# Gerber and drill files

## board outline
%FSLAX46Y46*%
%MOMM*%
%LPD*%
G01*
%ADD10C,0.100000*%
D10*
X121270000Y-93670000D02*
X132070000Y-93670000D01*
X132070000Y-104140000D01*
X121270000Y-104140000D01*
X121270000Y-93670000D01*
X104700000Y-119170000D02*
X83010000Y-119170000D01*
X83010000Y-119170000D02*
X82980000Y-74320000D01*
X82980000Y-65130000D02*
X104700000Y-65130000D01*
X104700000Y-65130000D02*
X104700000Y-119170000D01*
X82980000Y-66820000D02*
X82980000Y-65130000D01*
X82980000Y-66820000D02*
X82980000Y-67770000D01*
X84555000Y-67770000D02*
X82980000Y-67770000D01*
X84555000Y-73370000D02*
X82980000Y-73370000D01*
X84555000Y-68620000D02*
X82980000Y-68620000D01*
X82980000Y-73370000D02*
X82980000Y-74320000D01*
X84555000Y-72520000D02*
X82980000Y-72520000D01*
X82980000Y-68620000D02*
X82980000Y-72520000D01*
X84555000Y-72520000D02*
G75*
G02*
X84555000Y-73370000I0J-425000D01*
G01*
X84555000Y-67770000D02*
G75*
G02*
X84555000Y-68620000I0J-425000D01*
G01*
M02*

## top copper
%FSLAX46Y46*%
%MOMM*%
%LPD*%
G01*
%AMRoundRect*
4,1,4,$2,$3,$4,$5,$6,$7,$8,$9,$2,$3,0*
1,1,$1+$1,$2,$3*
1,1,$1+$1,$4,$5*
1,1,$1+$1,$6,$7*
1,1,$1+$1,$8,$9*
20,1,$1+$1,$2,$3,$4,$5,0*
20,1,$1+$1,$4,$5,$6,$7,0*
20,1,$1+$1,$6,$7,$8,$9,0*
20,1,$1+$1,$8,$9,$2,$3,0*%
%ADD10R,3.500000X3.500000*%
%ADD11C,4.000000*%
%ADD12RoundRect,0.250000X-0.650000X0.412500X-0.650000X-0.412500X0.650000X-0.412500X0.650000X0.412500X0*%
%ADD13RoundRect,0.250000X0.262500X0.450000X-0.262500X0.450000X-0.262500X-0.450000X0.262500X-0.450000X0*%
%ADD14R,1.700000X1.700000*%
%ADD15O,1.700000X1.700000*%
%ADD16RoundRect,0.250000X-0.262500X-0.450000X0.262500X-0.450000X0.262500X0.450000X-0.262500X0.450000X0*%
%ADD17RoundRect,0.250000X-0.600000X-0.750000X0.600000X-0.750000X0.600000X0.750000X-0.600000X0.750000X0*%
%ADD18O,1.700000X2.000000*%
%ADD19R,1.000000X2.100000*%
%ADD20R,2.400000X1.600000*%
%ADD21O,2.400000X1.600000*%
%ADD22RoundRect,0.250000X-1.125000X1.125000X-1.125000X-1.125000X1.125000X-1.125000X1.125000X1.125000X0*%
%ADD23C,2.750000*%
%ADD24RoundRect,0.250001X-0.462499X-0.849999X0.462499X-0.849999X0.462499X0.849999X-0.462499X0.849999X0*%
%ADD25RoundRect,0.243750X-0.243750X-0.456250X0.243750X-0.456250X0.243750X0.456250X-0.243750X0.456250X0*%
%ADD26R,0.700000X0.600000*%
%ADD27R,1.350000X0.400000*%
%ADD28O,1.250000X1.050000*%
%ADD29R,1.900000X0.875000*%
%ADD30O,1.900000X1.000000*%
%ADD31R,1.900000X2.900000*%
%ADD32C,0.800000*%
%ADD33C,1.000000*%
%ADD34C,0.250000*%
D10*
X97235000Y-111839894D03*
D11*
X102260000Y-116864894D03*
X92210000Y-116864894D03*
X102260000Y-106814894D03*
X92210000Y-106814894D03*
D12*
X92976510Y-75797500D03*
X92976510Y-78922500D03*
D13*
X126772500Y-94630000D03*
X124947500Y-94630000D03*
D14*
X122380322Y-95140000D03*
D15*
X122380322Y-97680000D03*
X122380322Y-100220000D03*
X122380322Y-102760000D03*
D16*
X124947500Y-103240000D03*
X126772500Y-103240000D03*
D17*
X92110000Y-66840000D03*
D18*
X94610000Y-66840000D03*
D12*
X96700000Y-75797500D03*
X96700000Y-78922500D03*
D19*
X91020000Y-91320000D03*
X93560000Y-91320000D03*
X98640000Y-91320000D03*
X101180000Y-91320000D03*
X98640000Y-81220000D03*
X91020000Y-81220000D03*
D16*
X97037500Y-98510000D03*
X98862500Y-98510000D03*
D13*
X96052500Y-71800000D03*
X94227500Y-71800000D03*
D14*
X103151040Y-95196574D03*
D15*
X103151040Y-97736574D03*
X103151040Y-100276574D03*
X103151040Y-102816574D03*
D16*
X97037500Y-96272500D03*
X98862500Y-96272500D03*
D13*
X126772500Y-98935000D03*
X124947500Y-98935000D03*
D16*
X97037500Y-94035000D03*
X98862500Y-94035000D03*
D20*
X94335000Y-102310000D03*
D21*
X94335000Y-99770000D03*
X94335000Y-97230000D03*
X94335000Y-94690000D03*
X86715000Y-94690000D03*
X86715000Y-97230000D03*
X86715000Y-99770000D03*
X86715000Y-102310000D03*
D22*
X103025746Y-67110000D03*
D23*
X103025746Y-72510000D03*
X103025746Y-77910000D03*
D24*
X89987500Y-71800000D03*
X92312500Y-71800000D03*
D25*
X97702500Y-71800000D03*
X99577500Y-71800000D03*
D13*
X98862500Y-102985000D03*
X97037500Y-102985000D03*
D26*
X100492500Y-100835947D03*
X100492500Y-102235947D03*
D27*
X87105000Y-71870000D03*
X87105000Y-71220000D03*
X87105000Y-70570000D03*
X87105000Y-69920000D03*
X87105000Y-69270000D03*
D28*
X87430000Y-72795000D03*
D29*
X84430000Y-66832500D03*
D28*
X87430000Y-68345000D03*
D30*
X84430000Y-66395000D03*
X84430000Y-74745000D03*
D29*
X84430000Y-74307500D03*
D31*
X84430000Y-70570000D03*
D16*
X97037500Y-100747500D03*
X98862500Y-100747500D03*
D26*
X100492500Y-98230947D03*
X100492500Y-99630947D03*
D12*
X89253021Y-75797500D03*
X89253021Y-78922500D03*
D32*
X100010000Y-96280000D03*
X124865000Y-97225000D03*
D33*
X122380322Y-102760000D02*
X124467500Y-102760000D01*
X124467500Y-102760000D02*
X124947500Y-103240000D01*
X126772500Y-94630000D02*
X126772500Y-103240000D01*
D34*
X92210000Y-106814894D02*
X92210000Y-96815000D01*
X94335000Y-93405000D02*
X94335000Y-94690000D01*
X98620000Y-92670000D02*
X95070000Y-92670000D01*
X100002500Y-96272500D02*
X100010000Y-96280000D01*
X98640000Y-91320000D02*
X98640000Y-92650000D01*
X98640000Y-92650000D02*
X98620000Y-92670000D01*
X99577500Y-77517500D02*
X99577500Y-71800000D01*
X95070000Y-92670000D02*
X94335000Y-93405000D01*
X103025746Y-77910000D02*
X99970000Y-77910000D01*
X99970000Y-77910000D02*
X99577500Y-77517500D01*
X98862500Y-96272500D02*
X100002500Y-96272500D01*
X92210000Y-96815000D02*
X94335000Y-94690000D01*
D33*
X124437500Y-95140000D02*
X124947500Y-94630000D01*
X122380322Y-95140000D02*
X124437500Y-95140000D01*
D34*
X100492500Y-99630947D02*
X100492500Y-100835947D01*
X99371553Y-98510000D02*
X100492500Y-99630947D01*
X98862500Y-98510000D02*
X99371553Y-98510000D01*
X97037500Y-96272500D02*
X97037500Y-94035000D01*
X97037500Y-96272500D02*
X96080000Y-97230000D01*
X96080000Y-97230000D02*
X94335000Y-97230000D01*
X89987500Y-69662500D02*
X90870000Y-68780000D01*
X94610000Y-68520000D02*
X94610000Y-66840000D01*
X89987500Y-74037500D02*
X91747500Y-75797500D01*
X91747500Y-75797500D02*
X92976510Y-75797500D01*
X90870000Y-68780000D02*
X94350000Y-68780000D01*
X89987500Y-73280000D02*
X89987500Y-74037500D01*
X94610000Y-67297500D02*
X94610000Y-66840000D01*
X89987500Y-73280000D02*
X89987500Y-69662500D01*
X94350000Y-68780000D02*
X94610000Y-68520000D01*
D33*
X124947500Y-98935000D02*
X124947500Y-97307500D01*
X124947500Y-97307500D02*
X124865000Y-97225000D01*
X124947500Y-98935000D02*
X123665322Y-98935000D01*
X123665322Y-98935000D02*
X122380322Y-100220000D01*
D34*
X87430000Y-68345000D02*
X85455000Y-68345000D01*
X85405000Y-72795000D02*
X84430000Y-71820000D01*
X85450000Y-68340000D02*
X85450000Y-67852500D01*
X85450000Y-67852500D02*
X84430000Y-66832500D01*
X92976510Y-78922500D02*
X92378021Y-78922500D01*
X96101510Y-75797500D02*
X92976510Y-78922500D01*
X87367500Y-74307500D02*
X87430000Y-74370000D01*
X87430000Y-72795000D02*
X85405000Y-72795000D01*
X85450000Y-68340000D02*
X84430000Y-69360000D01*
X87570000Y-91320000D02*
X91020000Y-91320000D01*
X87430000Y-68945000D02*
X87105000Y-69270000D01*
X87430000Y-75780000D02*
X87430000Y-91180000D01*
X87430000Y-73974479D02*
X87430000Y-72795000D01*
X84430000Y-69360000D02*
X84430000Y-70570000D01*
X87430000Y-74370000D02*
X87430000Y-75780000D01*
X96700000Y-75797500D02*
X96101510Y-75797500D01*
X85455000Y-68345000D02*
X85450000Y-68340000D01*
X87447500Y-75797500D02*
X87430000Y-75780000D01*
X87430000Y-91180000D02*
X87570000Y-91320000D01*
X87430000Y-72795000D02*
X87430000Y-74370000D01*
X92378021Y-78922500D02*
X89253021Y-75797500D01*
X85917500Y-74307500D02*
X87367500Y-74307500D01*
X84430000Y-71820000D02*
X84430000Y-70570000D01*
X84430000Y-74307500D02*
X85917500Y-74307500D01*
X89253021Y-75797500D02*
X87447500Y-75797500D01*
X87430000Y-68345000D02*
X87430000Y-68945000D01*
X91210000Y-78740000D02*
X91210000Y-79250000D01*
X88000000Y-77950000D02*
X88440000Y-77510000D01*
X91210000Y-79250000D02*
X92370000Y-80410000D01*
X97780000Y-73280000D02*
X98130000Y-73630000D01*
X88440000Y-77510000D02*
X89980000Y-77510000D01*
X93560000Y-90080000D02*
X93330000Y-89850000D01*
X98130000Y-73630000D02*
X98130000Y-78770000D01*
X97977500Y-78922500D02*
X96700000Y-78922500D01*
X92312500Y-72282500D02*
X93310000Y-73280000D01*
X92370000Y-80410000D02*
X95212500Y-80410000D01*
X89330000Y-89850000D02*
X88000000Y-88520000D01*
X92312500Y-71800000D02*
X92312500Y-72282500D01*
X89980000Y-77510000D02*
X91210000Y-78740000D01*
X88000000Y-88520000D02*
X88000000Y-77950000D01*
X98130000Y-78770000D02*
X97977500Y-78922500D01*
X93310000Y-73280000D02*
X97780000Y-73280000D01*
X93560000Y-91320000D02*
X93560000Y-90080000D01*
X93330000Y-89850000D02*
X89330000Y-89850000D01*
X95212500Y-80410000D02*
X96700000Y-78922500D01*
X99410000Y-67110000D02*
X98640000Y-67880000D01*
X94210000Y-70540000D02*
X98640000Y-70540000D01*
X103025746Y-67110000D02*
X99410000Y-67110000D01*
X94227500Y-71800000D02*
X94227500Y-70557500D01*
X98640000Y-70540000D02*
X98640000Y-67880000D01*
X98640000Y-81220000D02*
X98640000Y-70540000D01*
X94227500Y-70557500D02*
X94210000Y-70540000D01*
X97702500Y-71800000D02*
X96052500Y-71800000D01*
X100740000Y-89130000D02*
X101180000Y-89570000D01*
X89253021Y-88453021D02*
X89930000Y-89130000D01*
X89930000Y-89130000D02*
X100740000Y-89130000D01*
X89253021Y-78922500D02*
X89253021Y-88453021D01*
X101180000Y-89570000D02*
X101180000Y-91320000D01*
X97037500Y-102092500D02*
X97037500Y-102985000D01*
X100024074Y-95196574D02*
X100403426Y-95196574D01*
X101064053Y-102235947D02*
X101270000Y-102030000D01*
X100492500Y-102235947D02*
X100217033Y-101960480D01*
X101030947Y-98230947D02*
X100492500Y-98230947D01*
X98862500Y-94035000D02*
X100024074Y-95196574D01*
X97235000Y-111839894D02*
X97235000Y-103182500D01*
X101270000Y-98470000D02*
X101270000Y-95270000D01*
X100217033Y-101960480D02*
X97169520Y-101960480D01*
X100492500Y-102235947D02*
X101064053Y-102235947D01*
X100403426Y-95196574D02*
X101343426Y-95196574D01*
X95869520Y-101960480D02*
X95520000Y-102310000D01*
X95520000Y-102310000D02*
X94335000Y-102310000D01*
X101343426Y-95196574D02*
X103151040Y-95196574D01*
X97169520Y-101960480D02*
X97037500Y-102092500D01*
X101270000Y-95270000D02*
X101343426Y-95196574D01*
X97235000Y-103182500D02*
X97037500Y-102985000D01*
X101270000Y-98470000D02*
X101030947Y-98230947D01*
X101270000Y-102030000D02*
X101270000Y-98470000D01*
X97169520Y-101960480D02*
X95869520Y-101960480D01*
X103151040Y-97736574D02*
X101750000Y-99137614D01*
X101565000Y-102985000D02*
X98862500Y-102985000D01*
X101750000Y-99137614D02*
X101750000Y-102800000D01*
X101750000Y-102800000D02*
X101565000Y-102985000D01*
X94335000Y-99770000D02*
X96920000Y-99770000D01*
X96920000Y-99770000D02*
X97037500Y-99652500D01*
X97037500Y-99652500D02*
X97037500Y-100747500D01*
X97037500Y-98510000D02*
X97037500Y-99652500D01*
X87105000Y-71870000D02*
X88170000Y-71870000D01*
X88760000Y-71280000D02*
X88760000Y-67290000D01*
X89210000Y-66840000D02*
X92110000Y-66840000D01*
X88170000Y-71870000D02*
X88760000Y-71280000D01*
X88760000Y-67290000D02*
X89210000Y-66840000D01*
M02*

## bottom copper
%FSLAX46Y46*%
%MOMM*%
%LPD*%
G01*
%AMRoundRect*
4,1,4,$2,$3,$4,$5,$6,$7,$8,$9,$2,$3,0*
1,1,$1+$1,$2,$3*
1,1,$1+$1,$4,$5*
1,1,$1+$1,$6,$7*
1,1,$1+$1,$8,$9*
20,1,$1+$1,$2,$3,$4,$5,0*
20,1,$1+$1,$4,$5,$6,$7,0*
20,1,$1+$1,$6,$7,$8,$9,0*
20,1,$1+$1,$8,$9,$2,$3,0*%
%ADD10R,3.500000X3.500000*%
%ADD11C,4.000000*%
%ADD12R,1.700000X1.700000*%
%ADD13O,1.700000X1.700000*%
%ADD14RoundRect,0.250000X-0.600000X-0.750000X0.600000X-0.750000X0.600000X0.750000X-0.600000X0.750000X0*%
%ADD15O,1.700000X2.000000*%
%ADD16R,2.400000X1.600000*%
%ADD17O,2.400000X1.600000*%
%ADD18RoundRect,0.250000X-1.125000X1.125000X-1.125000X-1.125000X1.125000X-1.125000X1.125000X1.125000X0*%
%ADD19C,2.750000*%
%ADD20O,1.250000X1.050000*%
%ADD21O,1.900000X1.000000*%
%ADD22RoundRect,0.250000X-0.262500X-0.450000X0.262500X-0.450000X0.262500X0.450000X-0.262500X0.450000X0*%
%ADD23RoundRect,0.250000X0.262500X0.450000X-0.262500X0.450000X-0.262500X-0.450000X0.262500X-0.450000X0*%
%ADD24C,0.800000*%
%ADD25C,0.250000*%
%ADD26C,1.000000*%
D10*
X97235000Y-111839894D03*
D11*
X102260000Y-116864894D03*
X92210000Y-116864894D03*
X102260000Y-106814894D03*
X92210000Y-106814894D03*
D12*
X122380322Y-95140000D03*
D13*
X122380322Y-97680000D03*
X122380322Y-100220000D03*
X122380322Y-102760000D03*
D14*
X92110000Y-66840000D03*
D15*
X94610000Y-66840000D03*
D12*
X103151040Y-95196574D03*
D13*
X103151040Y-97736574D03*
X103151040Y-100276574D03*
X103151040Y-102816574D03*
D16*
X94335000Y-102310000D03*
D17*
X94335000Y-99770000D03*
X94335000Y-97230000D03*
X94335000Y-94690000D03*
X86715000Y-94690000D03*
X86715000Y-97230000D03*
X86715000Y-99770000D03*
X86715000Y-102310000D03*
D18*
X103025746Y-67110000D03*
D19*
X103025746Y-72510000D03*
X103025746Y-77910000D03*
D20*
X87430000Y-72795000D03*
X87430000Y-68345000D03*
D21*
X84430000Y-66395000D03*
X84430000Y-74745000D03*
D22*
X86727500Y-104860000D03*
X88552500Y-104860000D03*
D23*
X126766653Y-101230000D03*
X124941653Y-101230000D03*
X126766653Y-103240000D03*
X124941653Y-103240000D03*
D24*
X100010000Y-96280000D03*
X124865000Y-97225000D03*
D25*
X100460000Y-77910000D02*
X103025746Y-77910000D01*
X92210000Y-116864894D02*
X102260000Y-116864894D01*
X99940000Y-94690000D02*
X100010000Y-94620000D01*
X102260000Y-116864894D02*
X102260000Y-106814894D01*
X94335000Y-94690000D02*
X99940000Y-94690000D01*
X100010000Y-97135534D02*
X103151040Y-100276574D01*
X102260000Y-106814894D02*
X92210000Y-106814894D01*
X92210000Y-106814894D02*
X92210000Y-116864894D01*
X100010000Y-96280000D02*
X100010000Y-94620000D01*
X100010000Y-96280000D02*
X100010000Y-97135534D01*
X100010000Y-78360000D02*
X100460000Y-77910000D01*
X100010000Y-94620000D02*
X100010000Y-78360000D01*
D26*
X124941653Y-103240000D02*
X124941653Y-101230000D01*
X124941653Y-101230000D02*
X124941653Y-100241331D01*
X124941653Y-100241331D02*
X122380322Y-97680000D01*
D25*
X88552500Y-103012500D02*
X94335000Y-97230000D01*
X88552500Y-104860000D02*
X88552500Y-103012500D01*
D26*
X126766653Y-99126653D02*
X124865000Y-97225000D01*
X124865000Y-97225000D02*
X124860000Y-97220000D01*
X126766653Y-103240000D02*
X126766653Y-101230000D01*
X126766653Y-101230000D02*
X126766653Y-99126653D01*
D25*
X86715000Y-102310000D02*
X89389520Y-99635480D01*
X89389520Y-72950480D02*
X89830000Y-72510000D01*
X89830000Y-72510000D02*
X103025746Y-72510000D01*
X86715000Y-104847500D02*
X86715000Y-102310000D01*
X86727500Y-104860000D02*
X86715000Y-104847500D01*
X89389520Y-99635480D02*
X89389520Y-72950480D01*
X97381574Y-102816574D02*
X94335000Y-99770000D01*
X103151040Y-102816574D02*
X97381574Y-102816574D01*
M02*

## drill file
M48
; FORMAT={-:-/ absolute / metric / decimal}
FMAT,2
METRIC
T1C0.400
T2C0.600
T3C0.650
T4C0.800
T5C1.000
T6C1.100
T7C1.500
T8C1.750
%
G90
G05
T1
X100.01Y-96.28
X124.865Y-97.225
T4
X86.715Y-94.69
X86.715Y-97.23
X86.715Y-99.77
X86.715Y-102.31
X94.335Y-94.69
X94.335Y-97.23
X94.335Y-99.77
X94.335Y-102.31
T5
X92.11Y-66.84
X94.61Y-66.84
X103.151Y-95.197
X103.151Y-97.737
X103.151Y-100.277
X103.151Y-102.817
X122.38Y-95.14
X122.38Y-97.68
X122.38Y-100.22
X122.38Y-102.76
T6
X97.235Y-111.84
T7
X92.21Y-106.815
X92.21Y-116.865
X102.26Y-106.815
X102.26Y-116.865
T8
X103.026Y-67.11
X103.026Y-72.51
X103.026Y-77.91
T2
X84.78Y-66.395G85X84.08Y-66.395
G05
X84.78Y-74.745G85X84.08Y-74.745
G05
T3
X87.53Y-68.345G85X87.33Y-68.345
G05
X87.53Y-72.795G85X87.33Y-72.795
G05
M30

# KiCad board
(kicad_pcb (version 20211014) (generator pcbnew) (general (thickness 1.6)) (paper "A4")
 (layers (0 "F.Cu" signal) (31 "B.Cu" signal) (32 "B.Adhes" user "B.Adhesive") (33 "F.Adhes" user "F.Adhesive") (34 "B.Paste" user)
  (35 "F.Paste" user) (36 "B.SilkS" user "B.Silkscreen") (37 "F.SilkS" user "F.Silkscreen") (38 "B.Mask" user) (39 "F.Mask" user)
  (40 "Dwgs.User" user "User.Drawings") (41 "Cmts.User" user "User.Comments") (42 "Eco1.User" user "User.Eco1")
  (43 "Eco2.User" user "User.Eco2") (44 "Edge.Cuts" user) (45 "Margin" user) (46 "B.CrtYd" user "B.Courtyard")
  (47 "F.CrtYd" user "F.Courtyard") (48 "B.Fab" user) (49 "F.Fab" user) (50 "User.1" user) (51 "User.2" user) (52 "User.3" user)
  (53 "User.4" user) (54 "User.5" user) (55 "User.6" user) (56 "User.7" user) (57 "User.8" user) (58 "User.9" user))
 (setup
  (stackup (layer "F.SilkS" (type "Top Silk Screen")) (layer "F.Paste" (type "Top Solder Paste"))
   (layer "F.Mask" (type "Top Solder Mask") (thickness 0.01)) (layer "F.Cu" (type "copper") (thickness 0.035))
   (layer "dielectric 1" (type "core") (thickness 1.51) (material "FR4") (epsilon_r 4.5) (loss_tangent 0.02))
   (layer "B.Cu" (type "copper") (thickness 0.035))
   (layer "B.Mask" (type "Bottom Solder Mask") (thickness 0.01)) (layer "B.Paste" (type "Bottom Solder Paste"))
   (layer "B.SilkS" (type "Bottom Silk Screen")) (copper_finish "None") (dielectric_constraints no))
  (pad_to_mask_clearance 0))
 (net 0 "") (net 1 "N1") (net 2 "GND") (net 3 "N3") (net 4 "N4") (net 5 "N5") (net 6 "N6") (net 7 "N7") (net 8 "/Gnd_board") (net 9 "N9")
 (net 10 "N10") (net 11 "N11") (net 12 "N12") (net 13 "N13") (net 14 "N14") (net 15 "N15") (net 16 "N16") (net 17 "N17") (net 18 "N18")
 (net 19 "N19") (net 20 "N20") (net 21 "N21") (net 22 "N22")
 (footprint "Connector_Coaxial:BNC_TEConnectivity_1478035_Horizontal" (layer "F.Cu") (at 97.235 111.839894 -90)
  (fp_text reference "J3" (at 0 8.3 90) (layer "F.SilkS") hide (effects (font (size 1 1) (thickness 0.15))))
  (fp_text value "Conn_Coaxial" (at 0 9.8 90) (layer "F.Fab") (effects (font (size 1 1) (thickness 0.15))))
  (pad "1" thru_hole rect (at 0 0 270) (size 3.5 3.5) (drill 1.1) (layers *.Cu *.Mask) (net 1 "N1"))
  (pad "2" thru_hole circle (at 5.025 -5.025 270) (size 4 4) (drill 1.5) (layers *.Cu *.Mask) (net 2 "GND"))
  (pad "2" thru_hole circle (at 5.025 5.025 270) (size 4 4) (drill 1.5) (layers *.Cu *.Mask) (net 2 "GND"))
  (pad "2" thru_hole circle (at -5.025 -5.025 270) (size 4 4) (drill 1.5) (layers *.Cu *.Mask) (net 2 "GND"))
  (pad "2" thru_hole circle (at -5.025 5.025 270) (size 4 4) (drill 1.5) (layers *.Cu *.Mask) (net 2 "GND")))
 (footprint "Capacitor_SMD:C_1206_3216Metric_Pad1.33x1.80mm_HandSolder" (layer "F.Cu") (at 92.97651 77.36 -90)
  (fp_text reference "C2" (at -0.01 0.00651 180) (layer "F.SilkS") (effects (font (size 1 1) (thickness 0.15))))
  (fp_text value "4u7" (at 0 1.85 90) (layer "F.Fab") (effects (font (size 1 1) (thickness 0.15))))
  (pad "1" smd roundrect locked (at -1.5625 0 270) (size 1.325 1.8) (layers "F.Cu" "F.Paste" "F.Mask") (roundrect_rratio 0.188679)
   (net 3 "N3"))
  (pad "2" smd roundrect locked (at 1.5625 0 270) (size 1.325 1.8) (layers "F.Cu" "F.Paste" "F.Mask") (roundrect_rratio 0.188679)
   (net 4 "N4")))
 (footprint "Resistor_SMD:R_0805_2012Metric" (layer "F.Cu") (at 125.86 94.63 180)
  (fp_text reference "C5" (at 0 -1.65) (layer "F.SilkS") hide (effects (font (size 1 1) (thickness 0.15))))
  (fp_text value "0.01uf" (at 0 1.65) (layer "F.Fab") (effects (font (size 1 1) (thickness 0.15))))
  (pad "1" smd roundrect locked (at -0.9125 0 180) (size 1.025 1.4) (layers "F.Cu" "F.Paste" "F.Mask") (roundrect_rratio 0.243902)
   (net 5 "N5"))
  (pad "2" smd roundrect locked (at 0.9125 0 180) (size 1.025 1.4) (layers "F.Cu" "F.Paste" "F.Mask") (roundrect_rratio 0.243902)
   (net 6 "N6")))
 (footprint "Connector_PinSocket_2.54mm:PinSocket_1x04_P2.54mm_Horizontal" (layer "F.Cu") (at 122.380322 95.14)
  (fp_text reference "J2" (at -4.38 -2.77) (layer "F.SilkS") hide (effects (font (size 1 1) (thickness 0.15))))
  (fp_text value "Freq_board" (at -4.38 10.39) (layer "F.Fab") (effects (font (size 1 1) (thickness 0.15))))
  (pad "1" thru_hole rect locked (at 0 0) (size 1.7 1.7) (drill 1) (layers *.Cu *.Mask) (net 6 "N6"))
  (pad "2" thru_hole oval locked (at 0 2.54) (size 1.7 1.7) (drill 1) (layers *.Cu *.Mask) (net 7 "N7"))
  (pad "3" thru_hole oval locked (at 0 5.08) (size 1.7 1.7) (drill 1) (layers *.Cu *.Mask) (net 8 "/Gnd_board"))
  (pad "4" thru_hole oval locked (at 0 7.62) (size 1.7 1.7) (drill 1) (layers *.Cu *.Mask) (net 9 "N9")))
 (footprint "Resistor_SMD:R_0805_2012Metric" (layer "F.Cu") (at 125.86 103.24)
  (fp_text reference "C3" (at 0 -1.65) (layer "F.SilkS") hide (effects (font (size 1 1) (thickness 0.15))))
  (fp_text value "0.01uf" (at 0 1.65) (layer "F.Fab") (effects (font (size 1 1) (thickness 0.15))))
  (pad "1" smd roundrect locked (at -0.9125 0) (size 1.025 1.4) (layers "F.Cu" "F.Paste" "F.Mask") (roundrect_rratio 0.243902) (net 9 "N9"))
  (pad "2" smd roundrect locked (at 0.9125 0) (size 1.025 1.4) (layers "F.Cu" "F.Paste" "F.Mask") (roundrect_rratio 0.243902) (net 5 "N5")))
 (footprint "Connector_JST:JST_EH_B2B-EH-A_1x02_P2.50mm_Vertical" (layer "F.Cu") (at 92.11 66.84)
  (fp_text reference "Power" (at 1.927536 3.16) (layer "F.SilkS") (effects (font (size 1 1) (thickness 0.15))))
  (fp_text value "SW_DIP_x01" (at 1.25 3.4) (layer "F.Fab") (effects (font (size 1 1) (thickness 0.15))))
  (pad "1" thru_hole roundrect locked (at 0 0) (size 1.7 2) (drill 1) (layers *.Cu *.Mask) (roundrect_rratio 0.147059) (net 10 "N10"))
  (pad "2" thru_hole oval locked (at 2.5 0) (size 1.7 2) (drill 1) (layers *.Cu *.Mask) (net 3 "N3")))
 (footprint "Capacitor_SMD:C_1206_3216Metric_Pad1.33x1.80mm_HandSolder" (layer "F.Cu") (at 96.7 77.36 -90)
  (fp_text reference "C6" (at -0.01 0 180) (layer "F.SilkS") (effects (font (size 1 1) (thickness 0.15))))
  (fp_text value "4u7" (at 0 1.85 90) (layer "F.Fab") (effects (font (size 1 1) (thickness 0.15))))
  (pad "1" smd roundrect locked (at -1.5625 0 270) (size 1.325 1.8) (layers "F.Cu" "F.Paste" "F.Mask") (roundrect_rratio 0.188679)
   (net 4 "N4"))
  (pad "2" smd roundrect locked (at 1.5625 0 270) (size 1.325 1.8) (layers "F.Cu" "F.Paste" "F.Mask") (roundrect_rratio 0.188679)
   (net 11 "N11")))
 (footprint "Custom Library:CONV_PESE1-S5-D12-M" (layer "F.Cu") (at 96.1 86.27 90)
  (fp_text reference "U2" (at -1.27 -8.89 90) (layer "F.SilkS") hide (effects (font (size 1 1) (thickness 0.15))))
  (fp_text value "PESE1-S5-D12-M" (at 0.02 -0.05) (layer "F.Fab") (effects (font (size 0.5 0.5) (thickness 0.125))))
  (pad "1" smd rect (at -5.05 -5.08 90) (size 2.1 1) (layers "F.Cu" "F.Paste" "F.Mask") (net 4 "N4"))
  (pad "2" smd rect (at -5.05 -2.54 90) (size 2.1 1) (layers "F.Cu" "F.Paste" "F.Mask") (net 11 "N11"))
  (pad "4" smd rect (at -5.05 2.54 90) (size 2.1 1) (layers "F.Cu" "F.Paste" "F.Mask") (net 2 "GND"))
  (pad "5" smd rect (at -5.05 5.08 90) (size 2.1 1) (layers "F.Cu" "F.Paste" "F.Mask") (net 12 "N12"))
  (pad "7" smd rect (at 5.05 2.54 90) (size 2.1 1) (layers "F.Cu" "F.Paste" "F.Mask") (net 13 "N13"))
  (pad "10" smd rect (at 5.05 -5.08 90) (size 2.1 1) (layers "F.Cu" "F.Paste" "F.Mask")))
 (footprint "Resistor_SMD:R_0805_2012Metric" (layer "F.Cu") (at 97.95 98.51)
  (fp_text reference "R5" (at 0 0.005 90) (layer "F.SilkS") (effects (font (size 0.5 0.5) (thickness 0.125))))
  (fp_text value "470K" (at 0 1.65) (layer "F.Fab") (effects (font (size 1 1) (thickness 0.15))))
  (pad "1" smd roundrect locked (at -0.9125 0) (size 1.025 1.4) (layers "F.Cu" "F.Paste" "F.Mask") (roundrect_rratio 0.243902)
   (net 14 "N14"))
  (pad "2" smd roundrect locked (at 0.9125 0) (size 1.025 1.4) (layers "F.Cu" "F.Paste" "F.Mask") (roundrect_rratio 0.243902) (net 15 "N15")))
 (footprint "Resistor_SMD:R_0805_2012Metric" (layer "F.Cu") (at 95.14 71.8 180)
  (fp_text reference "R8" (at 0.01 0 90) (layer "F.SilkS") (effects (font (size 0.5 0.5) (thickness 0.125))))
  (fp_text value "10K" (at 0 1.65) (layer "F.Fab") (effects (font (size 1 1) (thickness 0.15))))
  (pad "1" smd roundrect locked (at -0.9125 0 180) (size 1.025 1.4) (layers "F.Cu" "F.Paste" "F.Mask") (roundrect_rratio 0.243902)
   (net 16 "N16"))
  (pad "2" smd roundrect locked (at 0.9125 0 180) (size 1.025 1.4) (layers "F.Cu" "F.Paste" "F.Mask") (roundrect_rratio 0.243902)
   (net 13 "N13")))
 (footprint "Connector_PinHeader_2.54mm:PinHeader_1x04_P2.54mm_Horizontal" (layer "F.Cu") (at 103.15104 95.196574)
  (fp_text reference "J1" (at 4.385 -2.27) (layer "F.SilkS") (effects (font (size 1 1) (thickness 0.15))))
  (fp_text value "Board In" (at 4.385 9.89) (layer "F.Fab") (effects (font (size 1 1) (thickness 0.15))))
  (pad "1" thru_hole rect locked (at 0 0) (size 1.7 1.7) (drill 1) (layers *.Cu *.Mask) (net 1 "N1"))
  (pad "2" thru_hole oval locked (at 0 2.54) (size 1.7 1.7) (drill 1) (layers *.Cu *.Mask) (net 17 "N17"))
  (pad "3" thru_hole oval locked (at 0 5.08) (size 1.7 1.7) (drill 1) (layers *.Cu *.Mask) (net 2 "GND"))
  (pad "4" thru_hole oval locked (at 0 7.62) (size 1.7 1.7) (drill 1) (layers *.Cu *.Mask) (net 14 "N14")))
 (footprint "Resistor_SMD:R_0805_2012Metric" (layer "F.Cu") (at 97.95 96.2725)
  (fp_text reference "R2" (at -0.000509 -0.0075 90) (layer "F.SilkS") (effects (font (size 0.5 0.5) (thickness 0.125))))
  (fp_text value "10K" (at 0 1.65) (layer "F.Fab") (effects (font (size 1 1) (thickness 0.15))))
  (pad "1" smd roundrect locked (at -0.9125 0) (size 1.025 1.4) (layers "F.Cu" "F.Paste" "F.Mask") (roundrect_rratio 0.243902)
   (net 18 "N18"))
  (pad "2" smd roundrect locked (at 0.9125 0) (size 1.025 1.4) (layers "F.Cu" "F.Paste" "F.Mask") (roundrect_rratio 0.243902) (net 2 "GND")))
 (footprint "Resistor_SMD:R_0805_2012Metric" (layer "F.Cu") (at 125.86 98.935 180)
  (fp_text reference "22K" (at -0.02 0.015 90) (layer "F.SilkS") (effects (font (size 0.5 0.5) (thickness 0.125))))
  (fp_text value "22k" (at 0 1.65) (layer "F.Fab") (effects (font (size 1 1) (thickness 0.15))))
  (pad "1" smd roundrect locked (at -0.9125 0 180) (size 1.025 1.4) (layers "F.Cu" "F.Paste" "F.Mask") (roundrect_rratio 0.243902)
   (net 5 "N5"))
  (pad "2" smd roundrect locked (at 0.9125 0 180) (size 1.025 1.4) (layers "F.Cu" "F.Paste" "F.Mask") (roundrect_rratio 0.243902)
   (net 8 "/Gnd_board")))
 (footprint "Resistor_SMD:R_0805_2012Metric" (layer "F.Cu") (at 97.95 94.035)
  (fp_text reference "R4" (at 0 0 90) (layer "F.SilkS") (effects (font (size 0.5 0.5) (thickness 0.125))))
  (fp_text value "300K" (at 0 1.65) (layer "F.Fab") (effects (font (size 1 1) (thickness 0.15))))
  (pad "1" smd roundrect locked (at -0.9125 0) (size 1.025 1.4) (layers "F.Cu" "F.Paste" "F.Mask") (roundrect_rratio 0.243902)
   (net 18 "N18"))
  (pad "2" smd roundrect locked (at 0.9125 0) (size 1.025 1.4) (layers "F.Cu" "F.Paste" "F.Mask") (roundrect_rratio 0.243902) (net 1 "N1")))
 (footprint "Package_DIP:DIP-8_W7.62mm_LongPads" (layer "F.Cu") (at 94.335 102.31 180)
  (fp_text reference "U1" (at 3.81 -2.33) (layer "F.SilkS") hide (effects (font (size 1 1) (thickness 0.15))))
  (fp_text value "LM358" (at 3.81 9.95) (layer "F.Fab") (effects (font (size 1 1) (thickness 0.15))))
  (pad "1" thru_hole rect locked (at 0 0 180) (size 2.4 1.6) (drill 0.8) (layers *.Cu *.Mask) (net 1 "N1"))
  (pad "2" thru_hole oval locked (at 0 2.54 180) (size 2.4 1.6) (drill 0.8) (layers *.Cu *.Mask) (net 14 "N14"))
  (pad "3" thru_hole oval locked (at 0 5.08 180) (size 2.4 1.6) (drill 0.8) (layers *.Cu *.Mask) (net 18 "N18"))
  (pad "4" thru_hole oval locked (at 0 7.62 180) (size 2.4 1.6) (drill 0.8) (layers *.Cu *.Mask) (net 2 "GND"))
  (pad "5" thru_hole oval locked (at 7.62 7.62 180) (size 2.4 1.6) (drill 0.8) (layers *.Cu *.Mask))
  (pad "6" thru_hole oval locked (at 7.62 5.08 180) (size 2.4 1.6) (drill 0.8) (layers *.Cu *.Mask))
  (pad "7" thru_hole oval locked (at 7.62 2.54 180) (size 2.4 1.6) (drill 0.8) (layers *.Cu *.Mask))
  (pad "8" thru_hole oval locked (at 7.62 0 180) (size 2.4 1.6) (drill 0.8) (layers *.Cu *.Mask) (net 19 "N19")))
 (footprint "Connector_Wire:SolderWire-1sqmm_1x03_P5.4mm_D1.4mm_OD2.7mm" (layer "F.Cu") (at 103.025746 67.11 -90)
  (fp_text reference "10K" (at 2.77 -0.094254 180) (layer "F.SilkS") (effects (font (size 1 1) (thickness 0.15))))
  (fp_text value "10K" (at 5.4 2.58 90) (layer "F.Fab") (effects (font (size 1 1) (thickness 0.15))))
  (pad "1" thru_hole roundrect locked (at 0 0 270) (size 2.75 2.75) (drill 1.75) (layers *.Cu *.Mask) (roundrect_rratio 0.090909)
   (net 13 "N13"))
  (pad "2" thru_hole circle locked (at 5.4 0 270) (size 2.75 2.75) (drill 1.75) (layers *.Cu *.Mask) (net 19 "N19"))
  (pad "3" thru_hole circle locked (at 10.8 0 270) (size 2.75 2.75) (drill 1.75) (layers *.Cu *.Mask) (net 2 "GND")))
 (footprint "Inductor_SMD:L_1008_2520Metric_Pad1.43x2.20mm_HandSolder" (layer "F.Cu") (at 91.15 71.8)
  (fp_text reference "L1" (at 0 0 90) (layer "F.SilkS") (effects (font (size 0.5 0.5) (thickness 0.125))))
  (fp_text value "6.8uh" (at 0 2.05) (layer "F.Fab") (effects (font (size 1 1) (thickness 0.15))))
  (pad "1" smd roundrect locked (at -1.1625 0) (size 1.425 2.2) (layers "F.Cu" "F.Paste" "F.Mask") (roundrect_rratio 0.175439) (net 3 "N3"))
  (pad "2" smd roundrect locked (at 1.1625 0) (size 1.425 2.2) (layers "F.Cu" "F.Paste" "F.Mask") (roundrect_rratio 0.175439) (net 11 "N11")))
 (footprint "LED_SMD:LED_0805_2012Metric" (layer "F.Cu") (at 98.64 71.8)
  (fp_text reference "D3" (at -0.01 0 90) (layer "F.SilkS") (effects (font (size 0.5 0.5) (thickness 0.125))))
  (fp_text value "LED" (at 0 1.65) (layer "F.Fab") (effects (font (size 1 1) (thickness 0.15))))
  (pad "1" smd roundrect locked (at -0.9375 0) (size 0.975 1.4) (layers "F.Cu" "F.Paste" "F.Mask") (roundrect_rratio 0.25) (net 16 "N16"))
  (pad "2" smd roundrect locked (at 0.9375 0) (size 0.975 1.4) (layers "F.Cu" "F.Paste" "F.Mask") (roundrect_rratio 0.25) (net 2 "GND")))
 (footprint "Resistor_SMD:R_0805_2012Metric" (layer "F.Cu") (at 97.95 102.985 180)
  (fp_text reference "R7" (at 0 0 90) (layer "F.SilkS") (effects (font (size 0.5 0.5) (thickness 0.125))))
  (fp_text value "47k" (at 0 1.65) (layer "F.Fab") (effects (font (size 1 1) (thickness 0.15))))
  (pad "1" smd roundrect locked (at -0.9125 0 180) (size 1.025 1.4) (layers "F.Cu" "F.Paste" "F.Mask") (roundrect_rratio 0.243902)
   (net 17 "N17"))
  (pad "2" smd roundrect locked (at 0.9125 0 180) (size 1.025 1.4) (layers "F.Cu" "F.Paste" "F.Mask") (roundrect_rratio 0.243902)
   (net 1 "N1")))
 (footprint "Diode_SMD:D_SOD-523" (layer "F.Cu") (at 100.4925 101.535947 -90)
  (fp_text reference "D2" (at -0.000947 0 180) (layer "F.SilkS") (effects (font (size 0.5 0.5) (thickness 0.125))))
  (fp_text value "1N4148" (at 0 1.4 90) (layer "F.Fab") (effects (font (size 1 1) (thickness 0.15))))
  (pad "1" smd rect locked (at -0.7 0 90) (size 0.6 0.7) (layers "F.Cu" "F.Paste" "F.Mask") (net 15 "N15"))
  (pad "2" smd rect locked (at 0.7 0 90) (size 0.6 0.7) (layers "F.Cu" "F.Paste" "F.Mask") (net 1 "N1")))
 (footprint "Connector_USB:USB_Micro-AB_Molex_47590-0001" (layer "F.Cu") (at 84.43 70.57 -90)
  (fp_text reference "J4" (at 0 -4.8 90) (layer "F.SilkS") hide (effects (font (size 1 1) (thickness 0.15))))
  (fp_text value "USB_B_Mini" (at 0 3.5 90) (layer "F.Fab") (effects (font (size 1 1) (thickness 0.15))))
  (fp_line (start -3.75 1.45) (end -2.8 1.45) (layer "Edge.Cuts") (width 0.1))
  (fp_line (start -2.8 -0.125) (end -2.8 1.45) (layer "Edge.Cuts") (width 0.1))
  (fp_line (start 2.8 -0.125) (end 2.8 1.45) (layer "Edge.Cuts") (width 0.1))
  (fp_line (start -1.95 -0.125) (end -1.95 1.45) (layer "Edge.Cuts") (width 0.1))
  (fp_line (start 2.8 1.45) (end 3.75 1.45) (layer "Edge.Cuts") (width 0.1))
  (fp_line (start 1.95 -0.125) (end 1.95 1.45) (layer "Edge.Cuts") (width 0.1))
  (fp_line (start -1.95 1.45) (end 1.95 1.45) (layer "Edge.Cuts") (width 0.1))
  (fp_arc (start 1.95 -0.125) (mid 2.375 -0.55) (end 2.8 -0.125) (layer "Edge.Cuts") (width 0.1))
  (fp_arc (start -2.8 -0.125) (mid -2.375 -0.55) (end -1.95 -0.125) (layer "Edge.Cuts") (width 0.1))
  (pad "" smd rect locked (at -3.5 0 270) (size 0.3 0.85) (layers "F.Paste"))
  (pad "" smd rect locked (at 3.5 0 270) (size 0.3 0.85) (layers "F.Paste"))
  (pad "1" smd rect locked (at 1.3 -2.675 270) (size 0.4 1.35) (layers "F.Cu" "F.Paste" "F.Mask") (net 10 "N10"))
  (pad "2" smd rect locked (at 0.65 -2.675 270) (size 0.4 1.35) (layers "F.Cu" "F.Paste" "F.Mask") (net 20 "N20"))
  (pad "3" smd rect locked (at 0 -2.675 270) (size 0.4 1.35) (layers "F.Cu" "F.Paste" "F.Mask") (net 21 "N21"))
  (pad "4" smd rect locked (at -0.65 -2.675 270) (size 0.4 1.35) (layers "F.Cu" "F.Paste" "F.Mask") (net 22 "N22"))
  (pad "5" smd rect locked (at -1.3 -2.675 270) (size 0.4 1.35) (layers "F.Cu" "F.Paste" "F.Mask") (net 4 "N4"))
  (pad "6" thru_hole oval locked (at 2.225 -3 270) (size 1.05 1.25) (drill oval 0.65 0.85) (layers *.Cu *.Mask) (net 4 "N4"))
  (pad "6" smd rect locked (at -3.7375 0 270) (size 0.875 1.9) (layers "F.Cu" "F.Mask") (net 4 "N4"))
  (pad "6" thru_hole oval locked (at -2.225 -3 270) (size 1.05 1.25) (drill oval 0.65 0.85) (layers *.Cu *.Mask) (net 4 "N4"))
  (pad "6" thru_hole oval locked (at -4.175 0 270) (size 1 1.9) (drill oval 0.6 1.3) (layers *.Cu *.Mask) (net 4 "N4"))
  (pad "6" thru_hole oval locked (at 4.175 0 270) (size 1 1.9) (drill oval 0.6 1.3) (layers *.Cu *.Mask) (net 4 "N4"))
  (pad "6" smd rect locked (at 3.7375 0 270) (size 0.875 1.9) (layers "F.Cu" "F.Mask") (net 4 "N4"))
  (pad "6" smd rect locked (at 0 0 270) (size 2.9 1.9) (layers "F.Cu" "F.Paste" "F.Mask") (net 4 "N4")))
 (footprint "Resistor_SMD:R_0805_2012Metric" (layer "F.Cu") (at 97.95 100.7475)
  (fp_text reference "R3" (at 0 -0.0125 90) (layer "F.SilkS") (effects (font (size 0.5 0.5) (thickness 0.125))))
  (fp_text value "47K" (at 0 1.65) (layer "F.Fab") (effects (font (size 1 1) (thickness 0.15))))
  (pad "1" smd roundrect locked (at -0.9125 0) (size 1.025 1.4) (layers "F.Cu" "F.Paste" "F.Mask") (roundrect_rratio 0.243902)
   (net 14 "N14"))
  (pad "2" smd roundrect locked (at 0.9125 0) (size 1.025 1.4) (layers "F.Cu" "F.Paste" "F.Mask") (roundrect_rratio 0.243902) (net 17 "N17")))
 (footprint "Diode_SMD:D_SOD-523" (layer "F.Cu") (at 100.4925 98.930947 -90)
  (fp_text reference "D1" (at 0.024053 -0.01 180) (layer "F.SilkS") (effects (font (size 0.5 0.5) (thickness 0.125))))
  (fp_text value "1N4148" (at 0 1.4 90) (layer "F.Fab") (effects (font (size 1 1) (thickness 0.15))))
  (pad "1" smd rect locked (at -0.7 0 90) (size 0.6 0.7) (layers "F.Cu" "F.Paste" "F.Mask") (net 1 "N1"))
  (pad "2" smd rect locked (at 0.7 0 90) (size 0.6 0.7) (layers "F.Cu" "F.Paste" "F.Mask") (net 15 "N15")))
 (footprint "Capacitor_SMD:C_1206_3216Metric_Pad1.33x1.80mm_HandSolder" (layer "F.Cu") (at 89.253021 77.36 -90)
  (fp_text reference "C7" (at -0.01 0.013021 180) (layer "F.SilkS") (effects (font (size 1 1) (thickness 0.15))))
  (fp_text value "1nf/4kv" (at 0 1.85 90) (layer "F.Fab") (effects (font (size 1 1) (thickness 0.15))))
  (pad "1" smd roundrect locked (at -1.5625 0 270) (size 1.325 1.8) (layers "F.Cu" "F.Paste" "F.Mask") (roundrect_rratio 0.188679)
   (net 4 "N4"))
  (pad "2" smd roundrect locked (at 1.5625 0 270) (size 1.325 1.8) (layers "F.Cu" "F.Paste" "F.Mask") (roundrect_rratio 0.188679)
   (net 12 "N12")))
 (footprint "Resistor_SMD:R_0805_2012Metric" (layer "B.Cu") (at 87.64 104.86)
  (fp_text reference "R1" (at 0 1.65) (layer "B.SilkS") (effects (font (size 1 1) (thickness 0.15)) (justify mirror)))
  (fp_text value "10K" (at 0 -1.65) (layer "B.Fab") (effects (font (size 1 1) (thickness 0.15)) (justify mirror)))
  (pad "1" smd roundrect locked (at -0.9125 0) (size 1.025 1.4) (layers "B.Cu" "B.Paste" "B.Mask") (roundrect_rratio 0.243902)
   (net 19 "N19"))
  (pad "2" smd roundrect locked (at 0.9125 0) (size 1.025 1.4) (layers "B.Cu" "B.Paste" "B.Mask") (roundrect_rratio 0.243902) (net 18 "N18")))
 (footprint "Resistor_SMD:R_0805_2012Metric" (layer "B.Cu") (at 125.854153 101.23 180)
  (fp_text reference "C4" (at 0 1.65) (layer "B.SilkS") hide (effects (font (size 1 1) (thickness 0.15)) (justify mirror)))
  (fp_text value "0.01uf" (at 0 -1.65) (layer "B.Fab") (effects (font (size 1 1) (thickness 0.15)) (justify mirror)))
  (pad "1" smd roundrect locked (at -0.9125 0 180) (size 1.025 1.4) (layers "B.Cu" "B.Paste" "B.Mask") (roundrect_rratio 0.243902)
   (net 8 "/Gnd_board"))
  (pad "2" smd roundrect locked (at 0.9125 0 180) (size 1.025 1.4) (layers "B.Cu" "B.Paste" "B.Mask") (roundrect_rratio 0.243902)
   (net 7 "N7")))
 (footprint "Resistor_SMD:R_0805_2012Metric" (layer "B.Cu") (at 125.854153 103.24 180)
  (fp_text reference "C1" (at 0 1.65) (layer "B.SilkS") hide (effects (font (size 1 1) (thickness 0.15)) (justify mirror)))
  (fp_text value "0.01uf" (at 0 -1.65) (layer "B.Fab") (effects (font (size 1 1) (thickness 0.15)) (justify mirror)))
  (pad "1" smd roundrect locked (at -0.9125 0 180) (size 1.025 1.4) (layers "B.Cu" "B.Paste" "B.Mask") (roundrect_rratio 0.243902)
   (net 8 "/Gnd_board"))
  (pad "2" smd roundrect locked (at 0.9125 0 180) (size 1.025 1.4) (layers "B.Cu" "B.Paste" "B.Mask") (roundrect_rratio 0.243902)
   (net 7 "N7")))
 (gr_rect (start 121.27 93.67) (end 132.07 104.14) (layer "Edge.Cuts") (width 0.1) (fill none))
 (gr_line (start 104.7 119.17) (end 83.01 119.17) (layer "Edge.Cuts") (width 0.1))
 (gr_line (start 83.01 119.17) (end 82.98 74.32) (layer "Edge.Cuts") (width 0.1))
 (gr_line (start 82.98 65.13) (end 104.7 65.13) (layer "Edge.Cuts") (width 0.1))
 (gr_line (start 104.7 65.13) (end 104.7 119.17) (layer "Edge.Cuts") (width 0.1))
 (gr_line (start 82.98 66.82) (end 82.98 65.13) (layer "Edge.Cuts") (width 0.1))
 (segment (start 122.380322 102.76) (end 124.4675 102.76) (width 1) (layer "F.Cu") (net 9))
 (segment (start 124.4675 102.76) (end 124.9475 103.24) (width 1) (layer "F.Cu") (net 9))
 (segment (start 126.7725 94.63) (end 126.7725 103.24) (width 1) (layer "F.Cu") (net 5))
 (segment (start 92.21 106.814894) (end 92.21 96.815) (width 0.25) (layer "F.Cu") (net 2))
 (segment (start 94.335 93.405) (end 94.335 94.69) (width 0.25) (layer "F.Cu") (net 2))
 (segment (start 98.62 92.67) (end 95.07 92.67) (width 0.25) (layer "F.Cu") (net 2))
 (segment (start 100.0025 96.2725) (end 100.01 96.28) (width 0.25) (layer "F.Cu") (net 2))
 (segment (start 98.64 91.32) (end 98.64 92.65) (width 0.25) (layer "F.Cu") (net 2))
 (segment (start 98.64 92.65) (end 98.62 92.67) (width 0.25) (layer "F.Cu") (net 2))
 (segment (start 99.5775 77.5175) (end 99.5775 71.8) (width 0.25) (layer "F.Cu") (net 2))
 (segment (start 95.07 92.67) (end 94.335 93.405) (width 0.25) (layer "F.Cu") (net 2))
 (segment (start 103.025746 77.91) (end 99.97 77.91) (width 0.25) (layer "F.Cu") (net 2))
 (segment (start 99.97 77.91) (end 99.5775 77.5175) (width 0.25) (layer "F.Cu") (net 2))
 (segment (start 98.8625 96.2725) (end 100.0025 96.2725) (width 0.25) (layer "F.Cu") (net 2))
 (segment (start 92.21 96.815) (end 94.335 94.69) (width 0.25) (layer "F.Cu") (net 2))
 (via (at 100.01 96.28) (size 0.8) (drill 0.4) (layers "F.Cu" "B.Cu") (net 2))
 (segment (start 100.46 77.91) (end 103.025746 77.91) (width 0.25) (layer "B.Cu") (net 2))
 (segment (start 92.21 116.864894) (end 102.26 116.864894) (width 0.25) (layer "B.Cu") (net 2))
 (segment (start 99.94 94.69) (end 100.01 94.62) (width 0.25) (layer "B.Cu") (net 2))
 (segment (start 102.26 116.864894) (end 102.26 106.814894) (width 0.25) (layer "B.Cu") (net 2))
 (segment (start 94.335 94.69) (end 99.94 94.69) (width 0.25) (layer "B.Cu") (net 2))
 (segment (start 100.01 97.135534) (end 103.15104 100.276574) (width 0.25) (layer "B.Cu") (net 2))
 (segment (start 102.26 106.814894) (end 92.21 106.814894) (width 0.25) (layer "B.Cu") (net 2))
 (segment (start 92.21 106.814894) (end 92.21 116.864894) (width 0.25) (layer "B.Cu") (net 2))
 (segment (start 100.01 96.28) (end 100.01 94.62) (width 0.25) (layer "B.Cu") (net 2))
 (segment (start 100.01 96.28) (end 100.01 97.135534) (width 0.25) (layer "B.Cu") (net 2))
 (segment (start 100.01 78.36) (end 100.46 77.91) (width 0.25) (layer "B.Cu") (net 2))
 (segment (start 100.01 94.62) (end 100.01 78.36) (width 0.25) (layer "B.Cu") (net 2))
 (segment (start 124.941653 103.24) (end 124.941653 101.23) (width 1) (layer "B.Cu") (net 7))
 (segment (start 124.941653 101.23) (end 124.941653 100.241331) (width 1) (layer "B.Cu") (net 7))
 (segment (start 124.941653 100.241331) (end 122.380322 97.68) (width 1) (layer "B.Cu") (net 7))
 (segment (start 124.4375 95.14) (end 124.9475 94.63) (width 1) (layer "F.Cu") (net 6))
 (segment (start 122.380322 95.14) (end 124.4375 95.14) (width 1) (layer "F.Cu") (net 6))
 (segment (start 100.4925 99.630947) (end 100.4925 100.835947) (width 0.25) (layer "F.Cu") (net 15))
 (segment (start 99.371553 98.51) (end 100.4925 99.630947) (width 0.25) (layer "F.Cu") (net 15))
 (segment (start 98.8625 98.51) (end 99.371553 98.51) (width 0.25) (layer "F.Cu") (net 15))
 (segment (start 97.0375 96.2725) (end 97.0375 94.035) (width 0.25) (layer "F.Cu") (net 18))
 (segment (start 97.0375 96.2725) (end 96.08 97.23) (width 0.25) (layer "F.Cu") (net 18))
 (segment (start 96.08 97.23) (end 94.335 97.23) (width 0.25) (layer "F.Cu") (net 18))
 (segment (start 88.5525 103.0125) (end 94.335 97.23) (width 0.25) (layer "B.Cu") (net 18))
 (segment (start 88.5525 104.86) (end 88.5525 103.0125) (width 0.25) (layer "B.Cu") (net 18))
 (segment (start 89.9875 69.6625) (end 90.87 68.78) (width 0.25) (layer "F.Cu") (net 3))
 (segment (start 94.61 68.52) (end 94.61 66.84) (width 0.25) (layer "F.Cu") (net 3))
 (segment (start 89.9875 74.0375) (end 91.7475 75.7975) (width 0.25) (layer "F.Cu") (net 3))
 (segment (start 91.7475 75.7975) (end 92.97651 75.7975) (width 0.25) (layer "F.Cu") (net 3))
 (segment (start 90.87 68.78) (end 94.35 68.78) (width 0.25) (layer "F.Cu") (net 3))
 (segment (start 89.9875 73.28) (end 89.9875 74.0375) (width 0.25) (layer "F.Cu") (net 3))
 (segment (start 94.61 67.2975) (end 94.61 66.84) (width 0.25) (layer "F.Cu") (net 3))
 (segment (start 89.9875 73.28) (end 89.9875 69.6625) (width 0.25) (layer "F.Cu") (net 3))
 (segment (start 94.35 68.78) (end 94.61 68.52) (width 0.25) (layer "F.Cu") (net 3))
 (segment (start 124.9475 98.935) (end 124.9475 97.3075) (width 1) (layer "F.Cu") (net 8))
 (segment (start 124.9475 97.3075) (end 124.865 97.225) (width 1) (layer "F.Cu") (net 8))
 (segment (start 124.9475 98.935) (end 123.665322 98.935) (width 1) (layer "F.Cu") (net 8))
 (segment (start 123.665322 98.935) (end 122.380322 100.22) (width 1) (layer "F.Cu") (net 8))
 (via (at 124.865 97.225) (size 0.8) (drill 0.4) (layers "F.Cu" "B.Cu") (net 8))
 (segment (start 126.766653 99.126653) (end 124.865 97.225) (width 1) (layer "B.Cu") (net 8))
 (segment (start 124.865 97.225) (end 124.86 97.22) (width 1) (layer "B.Cu") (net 8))
 (segment (start 126.766653 103.24) (end 126.766653 101.23) (width 1) (layer "B.Cu") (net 8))
 (segment (start 126.766653 101.23) (end 126.766653 99.126653) (width 1) (layer "B.Cu") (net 8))
 (segment (start 87.43 68.345) (end 85.455 68.345) (width 0.25) (layer "F.Cu") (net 4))
 (segment (start 85.405 72.795) (end 84.43 71.82) (width 0.25) (layer "F.Cu") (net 4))
 (segment (start 85.45 68.34) (end 85.45 67.8525) (width 0.25) (layer "F.Cu") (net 4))
 (segment (start 85.45 67.8525) (end 84.43 66.8325) (width 0.25) (layer "F.Cu") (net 4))
 (segment (start 92.97651 78.9225) (end 92.378021 78.9225) (width 0.25) (layer "F.Cu") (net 4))
 (segment (start 96.10151 75.7975) (end 92.97651 78.9225) (width 0.25) (layer "F.Cu") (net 4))
 (segment (start 87.3675 74.3075) (end 87.43 74.37) (width 0.25) (layer "F.Cu") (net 4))
 (segment (start 87.43 72.795) (end 85.405 72.795) (width 0.25) (layer "F.Cu") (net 4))
 (segment (start 85.45 68.34) (end 84.43 69.36) (width 0.25) (layer "F.Cu") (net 4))
 (segment (start 87.57 91.32) (end 91.02 91.32) (width 0.25) (layer "F.Cu") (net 4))
 (segment (start 87.43 68.945) (end 87.105 69.27) (width 0.25) (layer "F.Cu") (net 4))
 (segment (start 87.43 75.78) (end 87.43 91.18) (width 0.25) (layer "F.Cu") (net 4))
 (segment (start 87.43 73.974479) (end 87.43 72.795) (width 0.25) (layer "F.Cu") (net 4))
 (segment (start 84.43 69.36) (end 84.43 70.57) (width 0.25) (layer "F.Cu") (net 4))
 (segment (start 87.43 74.37) (end 87.43 75.78) (width 0.25) (layer "F.Cu") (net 4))
 (segment (start 96.7 75.7975) (end 96.10151 75.7975) (width 0.25) (layer "F.Cu") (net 4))
 (segment (start 85.455 68.345) (end 85.45 68.34) (width 0.25) (layer "F.Cu") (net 4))
 (segment (start 87.4475 75.7975) (end 87.43 75.78) (width 0.25) (layer "F.Cu") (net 4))
 (segment (start 87.43 91.18) (end 87.57 91.32) (width 0.25) (layer "F.Cu") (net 4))
 (segment (start 87.43 72.795) (end 87.43 74.37) (width 0.25) (layer "F.Cu") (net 4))
 (segment (start 92.378021 78.9225) (end 89.253021 75.7975) (width 0.25) (layer "F.Cu") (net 4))
 (segment (start 85.9175 74.3075) (end 87.3675 74.3075) (width 0.25) (layer "F.Cu") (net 4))
 (segment (start 84.43 71.82) (end 84.43 70.57) (width 0.25) (layer "F.Cu") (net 4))
 (segment (start 84.43 74.3075) (end 85.9175 74.3075) (width 0.25) (layer "F.Cu") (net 4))
 (segment (start 89.253021 75.7975) (end 87.4475 75.7975) (width 0.25) (layer "F.Cu") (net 4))
 (segment (start 87.43 68.345) (end 87.43 68.945) (width 0.25) (layer "F.Cu") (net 4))
 (segment (start 91.21 78.74) (end 91.21 79.25) (width 0.25) (layer "F.Cu") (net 11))
 (segment (start 88 77.95) (end 88.44 77.51) (width 0.25) (layer "F.Cu") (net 11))
 (segment (start 91.21 79.25) (end 92.37 80.41) (width 0.25) (layer "F.Cu") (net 11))
 (segment (start 97.78 73.28) (end 98.13 73.63) (width 0.25) (layer "F.Cu") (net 11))
 (segment (start 88.44 77.51) (end 89.98 77.51) (width 0.25) (layer "F.Cu") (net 11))
 (segment (start 93.56 90.08) (end 93.33 89.85) (width 0.25) (layer "F.Cu") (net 11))
 (segment (start 98.13 73.63) (end 98.13 78.77) (width 0.25) (layer "F.Cu") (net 11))
 (segment (start 97.9775 78.9225) (end 96.7 78.9225) (width 0.25) (layer "F.Cu") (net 11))
 (segment (start 92.3125 72.2825) (end 93.31 73.28) (width 0.25) (layer "F.Cu") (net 11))
 (segment (start 92.37 80.41) (end 95.2125 80.41) (width 0.25) (layer "F.Cu") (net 11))
 (segment (start 89.33 89.85) (end 88 88.52) (width 0.25) (layer "F.Cu") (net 11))
 (segment (start 92.3125 71.8) (end 92.3125 72.2825) (width 0.25) (layer "F.Cu") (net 11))
 (segment (start 89.98 77.51) (end 91.21 78.74) (width 0.25) (layer "F.Cu") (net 11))
 (segment (start 88 88.52) (end 88 77.95) (width 0.25) (layer "F.Cu") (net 11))
 (segment (start 98.13 78.77) (end 97.9775 78.9225) (width 0.25) (layer "F.Cu") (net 11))
 (segment (start 93.31 73.28) (end 97.78 73.28) (width 0.25) (layer "F.Cu") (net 11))
 (segment (start 93.56 91.32) (end 93.56 90.08) (width 0.25) (layer "F.Cu") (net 11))
 (segment (start 93.33 89.85) (end 89.33 89.85) (width 0.25) (layer "F.Cu") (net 11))
 (segment (start 95.2125 80.41) (end 96.7 78.9225) (width 0.25) (layer "F.Cu") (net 11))
 (segment (start 86.715 102.31) (end 89.38952 99.63548) (width 0.25) (layer "B.Cu") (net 19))
 (segment (start 89.38952 72.95048) (end 89.83 72.51) (width 0.25) (layer "B.Cu") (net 19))
 (segment (start 89.83 72.51) (end 103.025746 72.51) (width 0.25) (layer "B.Cu") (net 19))
 (segment (start 86.715 104.8475) (end 86.715 102.31) (width 0.25) (layer "B.Cu") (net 19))
 (segment (start 86.7275 104.86) (end 86.715 104.8475) (width 0.25) (layer "B.Cu") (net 19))
 (segment (start 89.38952 99.63548) (end 89.38952 72.95048) (width 0.25) (layer "B.Cu") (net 19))
 (segment (start 99.41 67.11) (end 98.64 67.88) (width 0.25) (layer "F.Cu") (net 13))
 (segment (start 94.21 70.54) (end 98.64 70.54) (width 0.25) (layer "F.Cu") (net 13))
 (segment (start 103.025746 67.11) (end 99.41 67.11) (width 0.25) (layer "F.Cu") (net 13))
 (segment (start 94.2275 71.8) (end 94.2275 70.5575) (width 0.25) (layer "F.Cu") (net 13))
 (segment (start 98.64 70.54) (end 98.64 67.88) (width 0.25) (layer "F.Cu") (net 13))
 (segment (start 98.64 81.22) (end 98.64 70.54) (width 0.25) (layer "F.Cu") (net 13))
 (segment (start 94.2275 70.5575) (end 94.21 70.54) (width 0.25) (layer "F.Cu") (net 13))
 (segment (start 97.7025 71.8) (end 96.0525 71.8) (width 0.25) (layer "F.Cu") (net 16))
 (segment (start 100.74 89.13) (end 101.18 89.57) (width 0.25) (layer "F.Cu") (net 12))
 (segment (start 89.253021 88.453021) (end 89.93 89.13) (width 0.25) (layer "F.Cu") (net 12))
 (segment (start 89.93 89.13) (end 100.74 89.13) (width 0.25) (layer "F.Cu") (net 12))
 (segment (start 89.253021 78.9225) (end 89.253021 88.453021) (width 0.25) (layer "F.Cu") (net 12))
 (segment (start 101.18 89.57) (end 101.18 91.32) (width 0.25) (layer "F.Cu") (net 12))
 (segment (start 97.0375 102.0925) (end 97.0375 102.985) (width 0.25) (layer "F.Cu") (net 1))
 (segment (start 100.024074 95.196574) (end 100.403426 95.196574) (width 0.25) (layer "F.Cu") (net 1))
 (segment (start 101.064053 102.235947) (end 101.27 102.03) (width 0.25) (layer "F.Cu") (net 1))
 (segment (start 100.4925 102.235947) (end 100.217033 101.96048) (width 0.25) (layer "F.Cu") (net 1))
 (segment (start 101.030947 98.230947) (end 100.4925 98.230947) (width 0.25) (layer "F.Cu") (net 1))
 (segment (start 98.8625 94.035) (end 100.024074 95.196574) (width 0.25) (layer "F.Cu") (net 1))
 (segment (start 97.235 111.839894) (end 97.235 103.1825) (width 0.25) (layer "F.Cu") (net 1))
 (segment (start 101.27 98.47) (end 101.27 95.27) (width 0.25) (layer "F.Cu") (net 1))
 (segment (start 100.217033 101.96048) (end 97.16952 101.96048) (width 0.25) (layer "F.Cu") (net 1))
 (segment (start 100.4925 102.235947) (end 101.064053 102.235947) (width 0.25) (layer "F.Cu") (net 1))
 (segment (start 100.403426 95.196574) (end 101.343426 95.196574) (width 0.25) (layer "F.Cu") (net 1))
 (segment (start 95.86952 101.96048) (end 95.52 102.31) (width 0.25) (layer "F.Cu") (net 1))
 (segment (start 95.52 102.31) (end 94.335 102.31) (width 0.25) (layer "F.Cu") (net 1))
 (segment (start 101.343426 95.196574) (end 103.15104 95.196574) (width 0.25) (layer "F.Cu") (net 1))
 (segment (start 97.16952 101.96048) (end 97.0375 102.0925) (width 0.25) (layer "F.Cu") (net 1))
 (segment (start 101.27 95.27) (end 101.343426 95.196574) (width 0.25) (layer "F.Cu") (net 1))
 (segment (start 97.235 103.1825) (end 97.0375 102.985) (width 0.25) (layer "F.Cu") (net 1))
 (segment (start 101.27 98.47) (end 101.030947 98.230947) (width 0.25) (layer "F.Cu") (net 1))
 (segment (start 101.27 102.03) (end 101.27 98.47) (width 0.25) (layer "F.Cu") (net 1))
 (segment (start 97.16952 101.96048) (end 95.86952 101.96048) (width 0.25) (layer "F.Cu") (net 1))
 (segment (start 103.15104 97.736574) (end 101.75 99.137614) (width 0.25) (layer "F.Cu") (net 17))
 (segment (start 101.565 102.985) (end 98.8625 102.985) (width 0.25) (layer "F.Cu") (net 17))
 (segment (start 101.75 99.137614) (end 101.75 102.8) (width 0.25) (layer "F.Cu") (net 17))
 (segment (start 101.75 102.8) (end 101.565 102.985) (width 0.25) (layer "F.Cu") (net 17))
 (segment (start 94.335 99.77) (end 96.92 99.77) (width 0.25) (layer "F.Cu") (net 14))
 (segment (start 96.92 99.77) (end 97.0375 99.6525) (width 0.25) (layer "F.Cu") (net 14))
 (segment (start 97.0375 99.6525) (end 97.0375 100.7475) (width 0.25) (layer "F.Cu") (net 14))
 (segment (start 97.0375 98.51) (end 97.0375 99.6525) (width 0.25) (layer "F.Cu") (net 14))
 (segment (start 97.381574 102.816574) (end 94.335 99.77) (width 0.25) (layer "B.Cu") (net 14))
 (segment (start 103.15104 102.816574) (end 97.381574 102.816574) (width 0.25) (layer "B.Cu") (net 14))
 (segment (start 87.105 71.87) (end 88.17 71.87) (width 0.25) (layer "F.Cu") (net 10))
 (segment (start 88.76 71.28) (end 88.76 67.29) (width 0.25) (layer "F.Cu") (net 10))
 (segment (start 89.21 66.84) (end 92.11 66.84) (width 0.25) (layer "F.Cu") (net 10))
 (segment (start 88.17 71.87) (end 88.76 71.28) (width 0.25) (layer "F.Cu") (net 10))
 (segment (start 88.76 67.29) (end 89.21 66.84) (width 0.25) (layer "F.Cu") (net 10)))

